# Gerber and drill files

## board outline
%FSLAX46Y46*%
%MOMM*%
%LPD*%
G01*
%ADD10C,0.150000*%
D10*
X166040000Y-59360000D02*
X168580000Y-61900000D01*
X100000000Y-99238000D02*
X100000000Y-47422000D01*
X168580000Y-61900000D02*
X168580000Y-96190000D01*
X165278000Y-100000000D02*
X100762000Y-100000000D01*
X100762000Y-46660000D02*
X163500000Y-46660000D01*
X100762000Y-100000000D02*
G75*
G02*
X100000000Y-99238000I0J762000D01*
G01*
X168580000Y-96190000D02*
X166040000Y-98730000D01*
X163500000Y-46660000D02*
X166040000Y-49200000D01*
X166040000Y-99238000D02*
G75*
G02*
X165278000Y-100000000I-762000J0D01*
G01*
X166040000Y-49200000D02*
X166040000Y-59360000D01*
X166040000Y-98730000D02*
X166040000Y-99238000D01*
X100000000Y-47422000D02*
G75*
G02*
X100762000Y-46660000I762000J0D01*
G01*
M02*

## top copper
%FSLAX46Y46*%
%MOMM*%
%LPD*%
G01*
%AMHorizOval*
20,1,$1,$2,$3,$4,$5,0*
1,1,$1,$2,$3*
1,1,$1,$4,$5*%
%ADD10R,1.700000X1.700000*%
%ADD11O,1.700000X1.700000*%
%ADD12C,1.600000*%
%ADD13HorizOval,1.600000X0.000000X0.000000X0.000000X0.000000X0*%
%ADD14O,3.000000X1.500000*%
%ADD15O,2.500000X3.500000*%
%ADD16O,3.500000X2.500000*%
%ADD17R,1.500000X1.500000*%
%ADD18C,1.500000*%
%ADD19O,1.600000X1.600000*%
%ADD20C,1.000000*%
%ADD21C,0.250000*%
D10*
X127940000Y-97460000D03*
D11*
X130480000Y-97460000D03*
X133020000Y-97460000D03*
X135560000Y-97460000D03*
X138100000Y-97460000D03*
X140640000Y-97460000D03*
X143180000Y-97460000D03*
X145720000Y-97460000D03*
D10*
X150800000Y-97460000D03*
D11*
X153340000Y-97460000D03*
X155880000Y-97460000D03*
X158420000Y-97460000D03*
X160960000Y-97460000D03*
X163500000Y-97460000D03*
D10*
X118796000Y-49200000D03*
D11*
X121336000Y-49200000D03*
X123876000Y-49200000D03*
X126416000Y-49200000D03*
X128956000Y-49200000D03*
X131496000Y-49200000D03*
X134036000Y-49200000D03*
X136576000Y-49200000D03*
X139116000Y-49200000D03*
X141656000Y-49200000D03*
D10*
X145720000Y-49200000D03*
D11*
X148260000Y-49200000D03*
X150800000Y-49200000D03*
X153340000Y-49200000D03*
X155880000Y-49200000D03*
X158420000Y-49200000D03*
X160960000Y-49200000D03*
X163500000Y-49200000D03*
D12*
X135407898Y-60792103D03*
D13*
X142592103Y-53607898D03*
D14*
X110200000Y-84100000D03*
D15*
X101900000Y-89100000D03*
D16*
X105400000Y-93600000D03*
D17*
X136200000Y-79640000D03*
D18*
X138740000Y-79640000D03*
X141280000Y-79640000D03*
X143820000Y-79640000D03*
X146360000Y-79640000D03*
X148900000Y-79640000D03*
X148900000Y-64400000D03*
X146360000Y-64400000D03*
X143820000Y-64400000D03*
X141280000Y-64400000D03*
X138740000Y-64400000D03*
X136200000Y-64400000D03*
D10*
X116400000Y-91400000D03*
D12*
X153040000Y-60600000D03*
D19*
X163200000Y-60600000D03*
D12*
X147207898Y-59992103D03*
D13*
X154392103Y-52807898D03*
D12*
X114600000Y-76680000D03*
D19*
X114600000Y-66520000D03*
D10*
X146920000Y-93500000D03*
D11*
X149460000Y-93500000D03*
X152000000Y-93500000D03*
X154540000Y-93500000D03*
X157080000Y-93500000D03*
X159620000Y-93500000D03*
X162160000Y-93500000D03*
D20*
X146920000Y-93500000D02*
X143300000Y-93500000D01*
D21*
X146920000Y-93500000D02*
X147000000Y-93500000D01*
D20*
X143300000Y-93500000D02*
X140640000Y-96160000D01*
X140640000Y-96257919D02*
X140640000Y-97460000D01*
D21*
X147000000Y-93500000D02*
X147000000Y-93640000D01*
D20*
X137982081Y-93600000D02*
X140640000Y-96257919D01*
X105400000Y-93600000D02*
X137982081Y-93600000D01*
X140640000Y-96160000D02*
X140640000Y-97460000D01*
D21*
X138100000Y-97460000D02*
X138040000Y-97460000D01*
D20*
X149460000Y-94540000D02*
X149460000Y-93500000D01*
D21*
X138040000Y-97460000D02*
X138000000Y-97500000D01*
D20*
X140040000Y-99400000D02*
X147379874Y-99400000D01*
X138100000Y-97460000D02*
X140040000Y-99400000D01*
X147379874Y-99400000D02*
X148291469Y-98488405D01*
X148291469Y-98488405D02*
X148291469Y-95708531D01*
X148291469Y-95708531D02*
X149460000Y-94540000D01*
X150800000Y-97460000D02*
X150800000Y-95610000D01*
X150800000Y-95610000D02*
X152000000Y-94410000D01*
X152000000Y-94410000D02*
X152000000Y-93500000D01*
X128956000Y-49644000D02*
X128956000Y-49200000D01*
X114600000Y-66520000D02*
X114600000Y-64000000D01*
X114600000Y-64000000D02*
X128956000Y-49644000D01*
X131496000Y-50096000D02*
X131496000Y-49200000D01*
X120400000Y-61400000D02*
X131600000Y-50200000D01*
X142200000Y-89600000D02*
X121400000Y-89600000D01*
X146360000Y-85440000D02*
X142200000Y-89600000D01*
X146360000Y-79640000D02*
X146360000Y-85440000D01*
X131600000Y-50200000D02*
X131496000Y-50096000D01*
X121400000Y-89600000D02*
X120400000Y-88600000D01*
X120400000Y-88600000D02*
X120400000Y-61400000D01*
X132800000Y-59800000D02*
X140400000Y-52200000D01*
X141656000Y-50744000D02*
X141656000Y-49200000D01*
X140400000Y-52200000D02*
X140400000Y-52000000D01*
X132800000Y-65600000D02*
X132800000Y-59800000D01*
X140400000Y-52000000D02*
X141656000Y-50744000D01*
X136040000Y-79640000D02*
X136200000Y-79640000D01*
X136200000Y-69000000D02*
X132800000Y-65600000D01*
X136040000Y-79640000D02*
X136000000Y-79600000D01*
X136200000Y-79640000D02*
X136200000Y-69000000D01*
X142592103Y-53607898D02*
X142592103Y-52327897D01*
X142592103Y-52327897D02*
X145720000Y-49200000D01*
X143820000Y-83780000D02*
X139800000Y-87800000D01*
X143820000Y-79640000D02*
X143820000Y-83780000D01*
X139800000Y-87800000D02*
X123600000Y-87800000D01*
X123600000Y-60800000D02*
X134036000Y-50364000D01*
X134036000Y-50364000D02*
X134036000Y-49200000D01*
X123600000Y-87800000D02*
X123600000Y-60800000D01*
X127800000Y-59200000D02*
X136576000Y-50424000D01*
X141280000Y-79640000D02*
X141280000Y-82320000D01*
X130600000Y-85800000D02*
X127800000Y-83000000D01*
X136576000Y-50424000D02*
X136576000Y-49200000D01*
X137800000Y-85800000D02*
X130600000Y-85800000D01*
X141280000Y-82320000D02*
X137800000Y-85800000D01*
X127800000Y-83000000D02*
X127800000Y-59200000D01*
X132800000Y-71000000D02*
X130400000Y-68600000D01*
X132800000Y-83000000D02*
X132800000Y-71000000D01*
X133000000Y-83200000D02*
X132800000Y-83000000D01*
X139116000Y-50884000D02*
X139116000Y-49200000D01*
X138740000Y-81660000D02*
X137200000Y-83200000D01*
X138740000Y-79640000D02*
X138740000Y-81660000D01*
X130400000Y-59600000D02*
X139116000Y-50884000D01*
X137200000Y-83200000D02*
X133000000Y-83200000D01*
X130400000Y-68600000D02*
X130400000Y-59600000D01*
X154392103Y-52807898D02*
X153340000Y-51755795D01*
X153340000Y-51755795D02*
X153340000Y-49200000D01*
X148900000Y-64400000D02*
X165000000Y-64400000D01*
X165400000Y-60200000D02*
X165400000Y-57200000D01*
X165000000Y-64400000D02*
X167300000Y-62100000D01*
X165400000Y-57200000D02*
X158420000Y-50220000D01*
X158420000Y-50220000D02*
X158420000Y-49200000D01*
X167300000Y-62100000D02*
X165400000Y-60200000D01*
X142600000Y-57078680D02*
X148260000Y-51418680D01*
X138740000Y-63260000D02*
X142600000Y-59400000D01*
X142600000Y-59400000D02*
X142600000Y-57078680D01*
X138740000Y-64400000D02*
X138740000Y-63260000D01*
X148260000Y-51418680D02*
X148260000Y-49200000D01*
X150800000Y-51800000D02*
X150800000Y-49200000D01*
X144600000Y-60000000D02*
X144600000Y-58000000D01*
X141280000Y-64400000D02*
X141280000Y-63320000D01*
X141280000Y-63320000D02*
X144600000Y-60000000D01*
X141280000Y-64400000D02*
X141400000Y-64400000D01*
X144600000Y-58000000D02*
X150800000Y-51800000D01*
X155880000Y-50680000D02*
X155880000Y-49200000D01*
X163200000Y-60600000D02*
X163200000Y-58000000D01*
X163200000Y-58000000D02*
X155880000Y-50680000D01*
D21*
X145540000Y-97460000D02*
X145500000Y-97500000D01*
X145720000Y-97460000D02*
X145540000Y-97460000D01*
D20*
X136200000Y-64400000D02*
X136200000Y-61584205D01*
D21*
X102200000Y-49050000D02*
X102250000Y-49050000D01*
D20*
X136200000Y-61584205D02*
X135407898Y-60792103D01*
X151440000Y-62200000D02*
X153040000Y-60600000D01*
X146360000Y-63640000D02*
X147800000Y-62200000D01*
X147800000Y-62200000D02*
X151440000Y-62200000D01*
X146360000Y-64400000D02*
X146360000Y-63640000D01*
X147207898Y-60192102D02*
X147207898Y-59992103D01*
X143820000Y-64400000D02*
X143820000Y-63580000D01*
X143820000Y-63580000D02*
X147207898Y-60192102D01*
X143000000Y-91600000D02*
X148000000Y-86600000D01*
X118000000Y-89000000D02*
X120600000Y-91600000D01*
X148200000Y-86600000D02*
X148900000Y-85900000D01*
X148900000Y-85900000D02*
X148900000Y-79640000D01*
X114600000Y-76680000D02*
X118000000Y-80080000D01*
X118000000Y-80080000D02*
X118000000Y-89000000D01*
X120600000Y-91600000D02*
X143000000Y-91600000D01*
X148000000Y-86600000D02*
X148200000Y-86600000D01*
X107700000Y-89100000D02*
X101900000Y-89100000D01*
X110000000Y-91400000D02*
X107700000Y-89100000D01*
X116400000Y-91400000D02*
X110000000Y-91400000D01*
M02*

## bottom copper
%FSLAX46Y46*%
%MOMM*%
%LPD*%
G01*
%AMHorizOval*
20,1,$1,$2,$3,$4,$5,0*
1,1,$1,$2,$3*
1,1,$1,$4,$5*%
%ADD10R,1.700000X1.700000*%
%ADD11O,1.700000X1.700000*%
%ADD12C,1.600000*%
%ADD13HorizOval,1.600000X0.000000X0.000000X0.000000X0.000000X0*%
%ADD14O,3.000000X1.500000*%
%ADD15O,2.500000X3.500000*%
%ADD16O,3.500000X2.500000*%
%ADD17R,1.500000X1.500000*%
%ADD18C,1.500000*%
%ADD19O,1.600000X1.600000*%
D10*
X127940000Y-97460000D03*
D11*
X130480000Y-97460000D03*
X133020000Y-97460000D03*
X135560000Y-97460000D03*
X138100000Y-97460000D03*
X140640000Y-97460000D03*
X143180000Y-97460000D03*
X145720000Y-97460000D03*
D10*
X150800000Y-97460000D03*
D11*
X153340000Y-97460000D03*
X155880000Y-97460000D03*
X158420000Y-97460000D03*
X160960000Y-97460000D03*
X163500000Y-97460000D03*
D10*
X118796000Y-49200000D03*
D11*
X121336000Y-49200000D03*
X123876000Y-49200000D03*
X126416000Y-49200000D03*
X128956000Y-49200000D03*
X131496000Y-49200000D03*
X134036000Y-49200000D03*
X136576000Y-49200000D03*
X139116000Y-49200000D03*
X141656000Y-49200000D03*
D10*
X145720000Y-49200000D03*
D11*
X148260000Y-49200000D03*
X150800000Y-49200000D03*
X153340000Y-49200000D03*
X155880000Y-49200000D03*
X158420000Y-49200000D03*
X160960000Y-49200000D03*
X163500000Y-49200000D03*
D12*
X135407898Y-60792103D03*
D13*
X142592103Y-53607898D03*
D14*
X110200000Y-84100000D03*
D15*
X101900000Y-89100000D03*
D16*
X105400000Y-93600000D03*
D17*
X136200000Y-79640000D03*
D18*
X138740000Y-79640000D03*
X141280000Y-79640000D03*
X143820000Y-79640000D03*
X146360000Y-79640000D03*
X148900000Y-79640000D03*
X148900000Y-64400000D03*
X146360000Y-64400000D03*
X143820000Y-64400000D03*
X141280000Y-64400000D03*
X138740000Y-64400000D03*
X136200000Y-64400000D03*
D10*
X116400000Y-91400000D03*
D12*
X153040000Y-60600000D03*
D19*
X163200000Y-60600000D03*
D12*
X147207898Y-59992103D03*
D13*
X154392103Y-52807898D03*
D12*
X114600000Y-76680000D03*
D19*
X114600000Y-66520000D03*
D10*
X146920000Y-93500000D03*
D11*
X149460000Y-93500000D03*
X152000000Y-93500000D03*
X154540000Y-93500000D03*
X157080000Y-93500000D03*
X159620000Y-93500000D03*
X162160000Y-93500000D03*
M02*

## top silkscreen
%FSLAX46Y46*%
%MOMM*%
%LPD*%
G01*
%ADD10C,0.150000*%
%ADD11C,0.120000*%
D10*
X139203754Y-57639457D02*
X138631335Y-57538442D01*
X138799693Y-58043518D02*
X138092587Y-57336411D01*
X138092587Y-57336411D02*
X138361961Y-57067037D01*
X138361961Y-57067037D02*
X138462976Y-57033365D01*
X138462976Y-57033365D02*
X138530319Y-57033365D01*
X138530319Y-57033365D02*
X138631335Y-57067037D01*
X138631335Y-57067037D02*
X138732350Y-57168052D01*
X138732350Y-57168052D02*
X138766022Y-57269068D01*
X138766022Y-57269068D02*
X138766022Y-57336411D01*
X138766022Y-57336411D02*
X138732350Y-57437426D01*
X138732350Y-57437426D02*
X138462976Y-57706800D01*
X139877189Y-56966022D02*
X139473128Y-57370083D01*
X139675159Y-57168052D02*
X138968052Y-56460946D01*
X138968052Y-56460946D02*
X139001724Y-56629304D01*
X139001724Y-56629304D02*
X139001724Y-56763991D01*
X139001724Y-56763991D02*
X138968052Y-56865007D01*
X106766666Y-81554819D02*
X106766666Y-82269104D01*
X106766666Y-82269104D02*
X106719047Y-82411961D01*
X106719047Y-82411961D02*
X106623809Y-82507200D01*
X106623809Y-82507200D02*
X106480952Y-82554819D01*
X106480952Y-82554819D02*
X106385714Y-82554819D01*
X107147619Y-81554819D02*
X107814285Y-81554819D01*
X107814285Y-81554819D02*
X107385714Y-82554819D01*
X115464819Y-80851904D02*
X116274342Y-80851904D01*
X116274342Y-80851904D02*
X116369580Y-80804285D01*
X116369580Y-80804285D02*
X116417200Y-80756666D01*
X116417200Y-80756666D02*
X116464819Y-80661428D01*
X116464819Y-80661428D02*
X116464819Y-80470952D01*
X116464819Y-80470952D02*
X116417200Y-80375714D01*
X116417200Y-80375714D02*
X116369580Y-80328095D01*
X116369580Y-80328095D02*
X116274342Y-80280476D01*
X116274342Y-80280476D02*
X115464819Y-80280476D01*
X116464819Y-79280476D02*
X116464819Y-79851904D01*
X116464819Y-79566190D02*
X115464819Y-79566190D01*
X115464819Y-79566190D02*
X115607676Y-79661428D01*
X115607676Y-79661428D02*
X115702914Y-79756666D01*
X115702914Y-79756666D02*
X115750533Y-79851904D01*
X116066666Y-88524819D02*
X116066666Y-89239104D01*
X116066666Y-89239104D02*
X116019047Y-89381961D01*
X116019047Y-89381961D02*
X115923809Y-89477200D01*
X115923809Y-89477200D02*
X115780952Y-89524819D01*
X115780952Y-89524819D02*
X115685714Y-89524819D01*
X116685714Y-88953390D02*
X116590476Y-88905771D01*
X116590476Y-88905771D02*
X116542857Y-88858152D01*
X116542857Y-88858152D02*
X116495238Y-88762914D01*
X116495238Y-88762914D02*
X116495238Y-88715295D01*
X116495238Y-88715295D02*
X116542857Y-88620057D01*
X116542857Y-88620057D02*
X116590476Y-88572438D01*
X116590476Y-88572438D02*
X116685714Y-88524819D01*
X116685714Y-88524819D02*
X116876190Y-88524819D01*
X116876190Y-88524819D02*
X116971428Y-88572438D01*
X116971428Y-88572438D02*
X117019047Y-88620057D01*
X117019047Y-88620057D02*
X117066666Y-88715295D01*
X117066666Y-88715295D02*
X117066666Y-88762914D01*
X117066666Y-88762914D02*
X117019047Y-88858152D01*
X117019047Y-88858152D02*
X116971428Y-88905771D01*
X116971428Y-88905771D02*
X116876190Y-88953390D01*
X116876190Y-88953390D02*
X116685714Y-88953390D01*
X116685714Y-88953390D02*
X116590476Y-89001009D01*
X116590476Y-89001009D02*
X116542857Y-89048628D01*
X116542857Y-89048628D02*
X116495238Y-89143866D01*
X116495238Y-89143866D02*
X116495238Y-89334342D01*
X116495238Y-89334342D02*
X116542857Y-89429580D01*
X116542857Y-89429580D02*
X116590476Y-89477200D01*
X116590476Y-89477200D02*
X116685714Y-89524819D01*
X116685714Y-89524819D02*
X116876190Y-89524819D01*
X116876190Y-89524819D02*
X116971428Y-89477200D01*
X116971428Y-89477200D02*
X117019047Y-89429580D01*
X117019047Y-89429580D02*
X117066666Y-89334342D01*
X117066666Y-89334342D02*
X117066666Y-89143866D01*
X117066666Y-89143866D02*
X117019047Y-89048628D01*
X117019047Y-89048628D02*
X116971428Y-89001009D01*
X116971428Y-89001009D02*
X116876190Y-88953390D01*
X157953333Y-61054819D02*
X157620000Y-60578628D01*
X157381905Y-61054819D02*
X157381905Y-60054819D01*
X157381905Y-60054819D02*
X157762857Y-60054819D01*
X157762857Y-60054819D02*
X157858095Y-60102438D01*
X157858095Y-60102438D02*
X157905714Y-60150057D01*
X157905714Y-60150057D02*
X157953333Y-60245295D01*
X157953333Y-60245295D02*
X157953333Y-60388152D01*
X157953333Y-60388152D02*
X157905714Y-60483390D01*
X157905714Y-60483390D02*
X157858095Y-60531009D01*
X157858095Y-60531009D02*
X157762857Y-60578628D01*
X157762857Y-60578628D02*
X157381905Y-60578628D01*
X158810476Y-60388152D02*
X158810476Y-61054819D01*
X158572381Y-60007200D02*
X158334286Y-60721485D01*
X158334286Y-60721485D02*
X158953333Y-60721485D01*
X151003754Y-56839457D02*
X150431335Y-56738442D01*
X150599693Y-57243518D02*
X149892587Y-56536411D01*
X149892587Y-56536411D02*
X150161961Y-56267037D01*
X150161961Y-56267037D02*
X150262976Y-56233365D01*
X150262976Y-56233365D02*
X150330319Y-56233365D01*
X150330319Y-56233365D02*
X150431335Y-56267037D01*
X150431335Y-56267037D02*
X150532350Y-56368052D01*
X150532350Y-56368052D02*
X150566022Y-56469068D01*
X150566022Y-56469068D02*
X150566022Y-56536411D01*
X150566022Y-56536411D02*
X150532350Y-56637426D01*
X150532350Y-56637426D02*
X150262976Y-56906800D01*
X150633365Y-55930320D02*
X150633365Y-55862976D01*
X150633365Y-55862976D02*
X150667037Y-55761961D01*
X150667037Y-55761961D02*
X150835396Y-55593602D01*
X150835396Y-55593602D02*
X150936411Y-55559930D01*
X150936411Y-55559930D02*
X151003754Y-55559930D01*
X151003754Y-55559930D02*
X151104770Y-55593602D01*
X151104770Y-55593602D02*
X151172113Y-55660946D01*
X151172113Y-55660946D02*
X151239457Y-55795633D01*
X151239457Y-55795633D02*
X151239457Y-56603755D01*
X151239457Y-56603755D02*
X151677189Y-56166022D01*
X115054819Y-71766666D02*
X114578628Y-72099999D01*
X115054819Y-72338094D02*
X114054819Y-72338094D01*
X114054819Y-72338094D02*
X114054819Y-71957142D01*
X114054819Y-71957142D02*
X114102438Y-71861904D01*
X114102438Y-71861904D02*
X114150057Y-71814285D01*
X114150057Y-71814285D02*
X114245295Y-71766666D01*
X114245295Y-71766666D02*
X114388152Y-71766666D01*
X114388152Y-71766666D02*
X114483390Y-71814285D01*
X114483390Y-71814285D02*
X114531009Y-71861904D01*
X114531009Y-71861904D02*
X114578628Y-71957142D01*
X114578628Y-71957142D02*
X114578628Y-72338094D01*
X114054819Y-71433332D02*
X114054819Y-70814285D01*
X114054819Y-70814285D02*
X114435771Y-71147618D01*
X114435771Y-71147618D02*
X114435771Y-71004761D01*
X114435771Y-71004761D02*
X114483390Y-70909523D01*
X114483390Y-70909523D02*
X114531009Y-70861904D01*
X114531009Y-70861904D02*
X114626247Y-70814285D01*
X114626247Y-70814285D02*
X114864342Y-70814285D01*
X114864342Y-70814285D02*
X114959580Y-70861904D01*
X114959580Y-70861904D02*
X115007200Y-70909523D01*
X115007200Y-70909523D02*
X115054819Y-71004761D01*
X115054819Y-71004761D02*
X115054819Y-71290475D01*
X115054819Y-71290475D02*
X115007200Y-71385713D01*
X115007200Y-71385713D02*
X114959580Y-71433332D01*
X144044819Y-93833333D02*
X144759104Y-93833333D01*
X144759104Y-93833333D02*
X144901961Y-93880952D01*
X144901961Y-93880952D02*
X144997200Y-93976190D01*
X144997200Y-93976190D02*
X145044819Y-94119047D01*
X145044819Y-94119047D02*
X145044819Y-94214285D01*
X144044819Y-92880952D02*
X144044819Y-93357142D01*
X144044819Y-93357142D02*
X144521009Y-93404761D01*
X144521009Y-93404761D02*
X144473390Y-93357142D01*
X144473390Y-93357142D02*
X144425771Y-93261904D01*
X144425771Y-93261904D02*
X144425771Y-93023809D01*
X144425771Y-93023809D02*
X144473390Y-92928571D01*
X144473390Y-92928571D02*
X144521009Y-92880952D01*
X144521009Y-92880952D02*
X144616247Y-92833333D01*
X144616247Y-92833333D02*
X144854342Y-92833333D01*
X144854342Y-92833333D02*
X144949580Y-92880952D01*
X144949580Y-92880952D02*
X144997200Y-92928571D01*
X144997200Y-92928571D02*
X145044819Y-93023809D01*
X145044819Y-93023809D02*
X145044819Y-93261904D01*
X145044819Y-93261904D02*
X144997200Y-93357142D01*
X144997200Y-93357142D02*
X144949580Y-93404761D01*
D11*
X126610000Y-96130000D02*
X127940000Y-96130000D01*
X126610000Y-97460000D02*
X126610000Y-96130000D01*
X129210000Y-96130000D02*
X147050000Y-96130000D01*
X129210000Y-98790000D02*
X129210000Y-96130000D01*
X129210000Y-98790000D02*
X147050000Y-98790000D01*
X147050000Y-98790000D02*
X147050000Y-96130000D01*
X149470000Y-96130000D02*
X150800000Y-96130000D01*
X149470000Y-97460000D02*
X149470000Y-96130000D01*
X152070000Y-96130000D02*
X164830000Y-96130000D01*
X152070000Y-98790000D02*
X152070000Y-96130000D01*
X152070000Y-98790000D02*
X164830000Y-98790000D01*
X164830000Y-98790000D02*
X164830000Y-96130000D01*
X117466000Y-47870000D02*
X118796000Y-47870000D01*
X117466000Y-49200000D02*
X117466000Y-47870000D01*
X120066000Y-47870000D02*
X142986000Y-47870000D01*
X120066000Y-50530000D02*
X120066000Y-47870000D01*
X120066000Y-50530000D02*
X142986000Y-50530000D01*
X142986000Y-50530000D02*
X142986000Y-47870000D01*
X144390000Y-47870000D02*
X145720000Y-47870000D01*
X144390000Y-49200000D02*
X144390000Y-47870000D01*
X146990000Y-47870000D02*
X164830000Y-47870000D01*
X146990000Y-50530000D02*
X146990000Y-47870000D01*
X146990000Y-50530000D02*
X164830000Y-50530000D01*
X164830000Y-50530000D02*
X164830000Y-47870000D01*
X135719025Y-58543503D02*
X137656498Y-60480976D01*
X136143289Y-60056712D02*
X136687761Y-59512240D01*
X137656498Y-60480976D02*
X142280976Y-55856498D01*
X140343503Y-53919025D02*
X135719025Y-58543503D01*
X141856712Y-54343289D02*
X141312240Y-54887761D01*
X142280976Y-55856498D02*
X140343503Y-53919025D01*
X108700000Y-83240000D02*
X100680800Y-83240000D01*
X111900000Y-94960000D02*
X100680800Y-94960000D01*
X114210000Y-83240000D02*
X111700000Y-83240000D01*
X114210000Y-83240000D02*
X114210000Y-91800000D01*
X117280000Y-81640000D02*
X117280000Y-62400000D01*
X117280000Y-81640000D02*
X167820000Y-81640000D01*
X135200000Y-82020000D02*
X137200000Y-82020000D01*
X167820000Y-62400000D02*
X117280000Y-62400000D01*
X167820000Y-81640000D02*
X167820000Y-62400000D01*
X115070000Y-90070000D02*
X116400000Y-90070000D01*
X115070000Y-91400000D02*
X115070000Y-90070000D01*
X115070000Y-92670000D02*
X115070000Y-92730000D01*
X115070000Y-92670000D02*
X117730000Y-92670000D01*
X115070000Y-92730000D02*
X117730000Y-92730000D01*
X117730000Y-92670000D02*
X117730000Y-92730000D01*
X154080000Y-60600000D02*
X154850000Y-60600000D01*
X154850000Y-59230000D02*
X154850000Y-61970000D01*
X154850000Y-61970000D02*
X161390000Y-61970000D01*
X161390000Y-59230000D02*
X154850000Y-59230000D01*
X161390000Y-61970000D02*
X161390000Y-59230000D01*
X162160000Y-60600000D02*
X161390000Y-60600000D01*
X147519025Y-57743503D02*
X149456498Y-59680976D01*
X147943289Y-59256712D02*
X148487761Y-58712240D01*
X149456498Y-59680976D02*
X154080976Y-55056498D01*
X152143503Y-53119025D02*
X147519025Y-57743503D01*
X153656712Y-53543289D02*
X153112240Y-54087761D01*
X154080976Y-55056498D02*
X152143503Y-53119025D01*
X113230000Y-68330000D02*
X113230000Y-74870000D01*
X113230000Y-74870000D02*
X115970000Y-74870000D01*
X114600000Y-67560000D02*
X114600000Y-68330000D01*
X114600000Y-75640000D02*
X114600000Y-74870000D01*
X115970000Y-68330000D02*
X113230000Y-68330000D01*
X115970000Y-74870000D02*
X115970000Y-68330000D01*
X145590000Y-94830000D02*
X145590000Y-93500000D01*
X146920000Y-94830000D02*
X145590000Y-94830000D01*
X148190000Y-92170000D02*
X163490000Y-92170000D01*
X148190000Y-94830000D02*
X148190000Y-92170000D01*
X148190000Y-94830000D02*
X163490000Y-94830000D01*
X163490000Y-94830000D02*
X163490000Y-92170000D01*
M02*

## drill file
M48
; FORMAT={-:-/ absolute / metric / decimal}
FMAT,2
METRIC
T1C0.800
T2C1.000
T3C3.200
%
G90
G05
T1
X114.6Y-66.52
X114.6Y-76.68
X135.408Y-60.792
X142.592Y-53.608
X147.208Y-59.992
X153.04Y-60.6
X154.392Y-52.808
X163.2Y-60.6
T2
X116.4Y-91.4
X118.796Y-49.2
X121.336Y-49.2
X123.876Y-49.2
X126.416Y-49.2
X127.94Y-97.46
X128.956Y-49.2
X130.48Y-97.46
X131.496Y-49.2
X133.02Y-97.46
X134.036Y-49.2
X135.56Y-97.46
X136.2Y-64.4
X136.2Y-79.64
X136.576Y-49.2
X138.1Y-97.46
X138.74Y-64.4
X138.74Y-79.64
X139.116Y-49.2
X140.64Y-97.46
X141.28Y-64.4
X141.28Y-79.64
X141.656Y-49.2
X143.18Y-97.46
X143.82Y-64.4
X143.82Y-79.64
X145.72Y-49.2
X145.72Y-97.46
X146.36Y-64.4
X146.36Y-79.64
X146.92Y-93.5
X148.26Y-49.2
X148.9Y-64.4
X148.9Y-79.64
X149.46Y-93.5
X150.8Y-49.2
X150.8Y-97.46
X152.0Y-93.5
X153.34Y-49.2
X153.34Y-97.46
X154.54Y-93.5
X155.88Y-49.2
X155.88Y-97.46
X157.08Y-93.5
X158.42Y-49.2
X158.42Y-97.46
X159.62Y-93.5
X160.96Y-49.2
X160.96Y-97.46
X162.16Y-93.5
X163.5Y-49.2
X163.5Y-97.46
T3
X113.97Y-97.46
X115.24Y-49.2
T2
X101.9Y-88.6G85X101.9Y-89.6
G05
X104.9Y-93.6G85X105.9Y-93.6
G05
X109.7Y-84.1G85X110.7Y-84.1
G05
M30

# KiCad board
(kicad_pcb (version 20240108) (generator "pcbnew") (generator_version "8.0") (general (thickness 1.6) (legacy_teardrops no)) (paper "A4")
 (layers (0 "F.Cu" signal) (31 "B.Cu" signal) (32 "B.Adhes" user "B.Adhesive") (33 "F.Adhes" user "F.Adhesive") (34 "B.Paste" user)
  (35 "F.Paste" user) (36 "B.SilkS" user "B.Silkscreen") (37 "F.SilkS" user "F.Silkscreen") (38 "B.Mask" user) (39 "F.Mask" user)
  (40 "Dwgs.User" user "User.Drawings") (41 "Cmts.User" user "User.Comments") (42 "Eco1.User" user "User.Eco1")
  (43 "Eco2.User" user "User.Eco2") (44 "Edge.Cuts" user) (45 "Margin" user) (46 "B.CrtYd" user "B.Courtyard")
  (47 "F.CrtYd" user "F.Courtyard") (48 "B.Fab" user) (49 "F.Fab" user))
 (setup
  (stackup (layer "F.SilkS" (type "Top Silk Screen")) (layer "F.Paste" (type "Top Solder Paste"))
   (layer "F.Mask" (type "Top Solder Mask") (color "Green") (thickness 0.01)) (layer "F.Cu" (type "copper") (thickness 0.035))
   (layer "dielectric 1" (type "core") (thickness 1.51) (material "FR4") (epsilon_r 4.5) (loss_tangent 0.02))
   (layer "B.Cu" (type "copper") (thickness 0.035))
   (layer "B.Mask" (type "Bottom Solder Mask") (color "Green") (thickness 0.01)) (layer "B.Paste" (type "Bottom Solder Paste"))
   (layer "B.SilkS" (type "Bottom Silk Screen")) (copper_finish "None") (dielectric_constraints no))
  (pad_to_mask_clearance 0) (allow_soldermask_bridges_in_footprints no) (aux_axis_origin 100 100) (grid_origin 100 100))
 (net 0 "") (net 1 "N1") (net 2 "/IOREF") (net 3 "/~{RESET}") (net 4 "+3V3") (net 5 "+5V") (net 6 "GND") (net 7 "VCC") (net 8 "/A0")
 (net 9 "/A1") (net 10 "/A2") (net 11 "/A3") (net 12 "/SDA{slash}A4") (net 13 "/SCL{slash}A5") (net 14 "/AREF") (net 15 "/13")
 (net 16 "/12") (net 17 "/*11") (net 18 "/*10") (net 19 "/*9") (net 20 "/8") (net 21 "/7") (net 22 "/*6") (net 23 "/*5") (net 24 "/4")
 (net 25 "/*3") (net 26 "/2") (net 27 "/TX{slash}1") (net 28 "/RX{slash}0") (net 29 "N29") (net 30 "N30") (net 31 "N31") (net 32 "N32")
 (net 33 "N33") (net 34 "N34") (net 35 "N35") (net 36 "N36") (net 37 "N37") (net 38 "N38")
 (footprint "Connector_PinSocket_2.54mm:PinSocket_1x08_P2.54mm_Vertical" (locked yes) (layer "F.Cu") (at 127.94 97.46 90)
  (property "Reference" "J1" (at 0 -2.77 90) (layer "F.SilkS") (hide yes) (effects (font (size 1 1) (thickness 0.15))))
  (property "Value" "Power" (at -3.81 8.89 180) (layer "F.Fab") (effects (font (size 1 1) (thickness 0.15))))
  (fp_line (start 1.33 -1.33) (end 1.33 0) (stroke (width 0.12) (type solid)) (layer "F.SilkS"))
  (fp_line (start 0 -1.33) (end 1.33 -1.33) (stroke (width 0.12) (type solid)) (layer "F.SilkS"))
  (fp_line (start 1.33 1.27) (end 1.33 19.11) (stroke (width 0.12) (type solid)) (layer "F.SilkS"))
  (fp_line (start -1.33 1.27) (end 1.33 1.27) (stroke (width 0.12) (type solid)) (layer "F.SilkS"))
  (fp_line (start -1.33 1.27) (end -1.33 19.11) (stroke (width 0.12) (type solid)) (layer "F.SilkS"))
  (fp_line (start -1.33 19.11) (end 1.33 19.11) (stroke (width 0.12) (type solid)) (layer "F.SilkS"))
  (pad "1" thru_hole rect (at 0 0 90) (size 1.7 1.7) (drill 1) (layers "*.Cu" "*.Mask") (remove_unused_layers no) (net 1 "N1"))
  (pad "2" thru_hole oval (at 0 2.54 90) (size 1.7 1.7) (drill 1) (layers "*.Cu" "*.Mask") (remove_unused_layers no) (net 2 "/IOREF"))
  (pad "3" thru_hole oval (at 0 5.08 90) (size 1.7 1.7) (drill 1) (layers "*.Cu" "*.Mask") (remove_unused_layers no) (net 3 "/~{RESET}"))
  (pad "4" thru_hole oval (at 0 7.62 90) (size 1.7 1.7) (drill 1) (layers "*.Cu" "*.Mask") (remove_unused_layers no) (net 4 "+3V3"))
  (pad "5" thru_hole oval (at 0 10.16 90) (size 1.7 1.7) (drill 1) (layers "*.Cu" "*.Mask") (remove_unused_layers no) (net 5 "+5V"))
  (pad "6" thru_hole oval (at 0 12.7 90) (size 1.7 1.7) (drill 1) (layers "*.Cu" "*.Mask") (remove_unused_layers no) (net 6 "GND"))
  (pad "7" thru_hole oval (at 0 15.24 90) (size 1.7 1.7) (drill 1) (layers "*.Cu" "*.Mask") (remove_unused_layers no) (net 6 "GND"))
  (pad "8" thru_hole oval (at 0 17.78 90) (size 1.7 1.7) (drill 1) (layers "*.Cu" "*.Mask") (remove_unused_layers no) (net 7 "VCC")))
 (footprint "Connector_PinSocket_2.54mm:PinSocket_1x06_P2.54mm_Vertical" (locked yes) (layer "F.Cu") (at 150.8 97.46 90)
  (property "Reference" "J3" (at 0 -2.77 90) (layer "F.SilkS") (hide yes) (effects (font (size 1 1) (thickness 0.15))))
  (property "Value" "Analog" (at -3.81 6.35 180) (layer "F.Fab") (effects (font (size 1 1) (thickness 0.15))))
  (fp_line (start 1.33 -1.33) (end 1.33 0) (stroke (width 0.12) (type solid)) (layer "F.SilkS"))
  (fp_line (start 0 -1.33) (end 1.33 -1.33) (stroke (width 0.12) (type solid)) (layer "F.SilkS"))
  (fp_line (start 1.33 1.27) (end 1.33 14.03) (stroke (width 0.12) (type solid)) (layer "F.SilkS"))
  (fp_line (start -1.33 1.27) (end 1.33 1.27) (stroke (width 0.12) (type solid)) (layer "F.SilkS"))
  (fp_line (start -1.33 1.27) (end -1.33 14.03) (stroke (width 0.12) (type solid)) (layer "F.SilkS"))
  (fp_line (start -1.33 14.03) (end 1.33 14.03) (stroke (width 0.12) (type solid)) (layer "F.SilkS"))
  (pad "1" thru_hole rect (at 0 0 90) (size 1.7 1.7) (drill 1) (layers "*.Cu" "*.Mask") (remove_unused_layers no) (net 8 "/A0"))
  (pad "2" thru_hole oval (at 0 2.54 90) (size 1.7 1.7) (drill 1) (layers "*.Cu" "*.Mask") (remove_unused_layers no) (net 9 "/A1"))
  (pad "3" thru_hole oval (at 0 5.08 90) (size 1.7 1.7) (drill 1) (layers "*.Cu" "*.Mask") (remove_unused_layers no) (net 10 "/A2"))
  (pad "4" thru_hole oval (at 0 7.62 90) (size 1.7 1.7) (drill 1) (layers "*.Cu" "*.Mask") (remove_unused_layers no) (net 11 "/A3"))
  (pad "5" thru_hole oval (at 0 10.16 90) (size 1.7 1.7) (drill 1) (layers "*.Cu" "*.Mask") (remove_unused_layers no)
   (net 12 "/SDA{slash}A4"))
  (pad "6" thru_hole oval (at 0 12.7 90) (size 1.7 1.7) (drill 1) (layers "*.Cu" "*.Mask") (remove_unused_layers no)
   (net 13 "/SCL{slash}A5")))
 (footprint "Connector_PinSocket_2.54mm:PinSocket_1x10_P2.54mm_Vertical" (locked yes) (layer "F.Cu") (at 118.796 49.2 90)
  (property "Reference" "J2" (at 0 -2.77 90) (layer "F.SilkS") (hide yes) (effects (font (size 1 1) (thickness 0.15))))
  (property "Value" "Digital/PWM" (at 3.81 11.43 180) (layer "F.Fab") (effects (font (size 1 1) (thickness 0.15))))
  (fp_line (start 1.33 -1.33) (end 1.33 0) (stroke (width 0.12) (type solid)) (layer "F.SilkS"))
  (fp_line (start 0 -1.33) (end 1.33 -1.33) (stroke (width 0.12) (type solid)) (layer "F.SilkS"))
  (fp_line (start 1.33 1.27) (end 1.33 24.19) (stroke (width 0.12) (type solid)) (layer "F.SilkS"))
  (fp_line (start -1.33 1.27) (end 1.33 1.27) (stroke (width 0.12) (type solid)) (layer "F.SilkS"))
  (fp_line (start -1.33 1.27) (end -1.33 24.19) (stroke (width 0.12) (type solid)) (layer "F.SilkS"))
  (fp_line (start -1.33 24.19) (end 1.33 24.19) (stroke (width 0.12) (type solid)) (layer "F.SilkS"))
  (pad "1" thru_hole rect (at 0 0 90) (size 1.7 1.7) (drill 1) (layers "*.Cu" "*.Mask") (remove_unused_layers no) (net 13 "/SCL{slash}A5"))
  (pad "2" thru_hole oval (at 0 2.54 90) (size 1.7 1.7) (drill 1) (layers "*.Cu" "*.Mask") (remove_unused_layers no)
   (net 12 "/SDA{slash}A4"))
  (pad "3" thru_hole oval (at 0 5.08 90) (size 1.7 1.7) (drill 1) (layers "*.Cu" "*.Mask") (remove_unused_layers no) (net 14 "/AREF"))
  (pad "4" thru_hole oval (at 0 7.62 90) (size 1.7 1.7) (drill 1) (layers "*.Cu" "*.Mask") (remove_unused_layers no) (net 6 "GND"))
  (pad "5" thru_hole oval (at 0 10.16 90) (size 1.7 1.7) (drill 1) (layers "*.Cu" "*.Mask") (remove_unused_layers no) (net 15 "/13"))
  (pad "6" thru_hole oval (at 0 12.7 90) (size 1.7 1.7) (drill 1) (layers "*.Cu" "*.Mask") (remove_unused_layers no) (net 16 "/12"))
  (pad "7" thru_hole oval (at 0 15.24 90) (size 1.7 1.7) (drill 1) (layers "*.Cu" "*.Mask") (remove_unused_layers no) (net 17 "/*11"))
  (pad "8" thru_hole oval (at 0 17.78 90) (size 1.7 1.7) (drill 1) (layers "*.Cu" "*.Mask") (remove_unused_layers no) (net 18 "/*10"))
  (pad "9" thru_hole oval (at 0 20.32 90) (size 1.7 1.7) (drill 1) (layers "*.Cu" "*.Mask") (remove_unused_layers no) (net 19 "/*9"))
  (pad "10" thru_hole oval (at 0 22.86 90) (size 1.7 1.7) (drill 1) (layers "*.Cu" "*.Mask") (remove_unused_layers no) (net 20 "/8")))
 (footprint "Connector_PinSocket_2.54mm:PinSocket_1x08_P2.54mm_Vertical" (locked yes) (layer "F.Cu") (at 145.72 49.2 90)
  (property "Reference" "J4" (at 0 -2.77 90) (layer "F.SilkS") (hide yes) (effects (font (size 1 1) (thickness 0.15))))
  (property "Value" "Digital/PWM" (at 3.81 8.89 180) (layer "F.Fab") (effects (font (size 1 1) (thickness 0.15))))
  (fp_line (start 1.33 -1.33) (end 1.33 0) (stroke (width 0.12) (type solid)) (layer "F.SilkS"))
  (fp_line (start 0 -1.33) (end 1.33 -1.33) (stroke (width 0.12) (type solid)) (layer "F.SilkS"))
  (fp_line (start 1.33 1.27) (end 1.33 19.11) (stroke (width 0.12) (type solid)) (layer "F.SilkS"))
  (fp_line (start -1.33 1.27) (end 1.33 1.27) (stroke (width 0.12) (type solid)) (layer "F.SilkS"))
  (fp_line (start -1.33 1.27) (end -1.33 19.11) (stroke (width 0.12) (type solid)) (layer "F.SilkS"))
  (fp_line (start -1.33 19.11) (end 1.33 19.11) (stroke (width 0.12) (type solid)) (layer "F.SilkS"))
  (pad "1" thru_hole rect (at 0 0 90) (size 1.7 1.7) (drill 1) (layers "*.Cu" "*.Mask") (remove_unused_layers no) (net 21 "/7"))
  (pad "2" thru_hole oval (at 0 2.54 90) (size 1.7 1.7) (drill 1) (layers "*.Cu" "*.Mask") (remove_unused_layers no) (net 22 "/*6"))
  (pad "3" thru_hole oval (at 0 5.08 90) (size 1.7 1.7) (drill 1) (layers "*.Cu" "*.Mask") (remove_unused_layers no) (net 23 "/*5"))
  (pad "4" thru_hole oval (at 0 7.62 90) (size 1.7 1.7) (drill 1) (layers "*.Cu" "*.Mask") (remove_unused_layers no) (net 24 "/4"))
  (pad "5" thru_hole oval (at 0 10.16 90) (size 1.7 1.7) (drill 1) (layers "*.Cu" "*.Mask") (remove_unused_layers no) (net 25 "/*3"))
  (pad "6" thru_hole oval (at 0 12.7 90) (size 1.7 1.7) (drill 1) (layers "*.Cu" "*.Mask") (remove_unused_layers no) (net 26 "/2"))
  (pad "7" thru_hole oval (at 0 15.24 90) (size 1.7 1.7) (drill 1) (layers "*.Cu" "*.Mask") (remove_unused_layers no) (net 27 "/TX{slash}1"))
  (pad "8" thru_hole oval (at 0 17.78 90) (size 1.7 1.7) (drill 1) (layers "*.Cu" "*.Mask") (remove_unused_layers no) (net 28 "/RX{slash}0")))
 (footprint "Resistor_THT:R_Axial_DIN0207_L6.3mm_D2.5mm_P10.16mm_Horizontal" (layer "F.Cu") (at 135.407898 60.792103 45)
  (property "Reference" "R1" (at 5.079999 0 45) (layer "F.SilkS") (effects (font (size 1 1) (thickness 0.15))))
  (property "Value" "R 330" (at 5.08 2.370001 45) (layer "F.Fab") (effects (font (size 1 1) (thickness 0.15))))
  (fp_line (start 1.81 -1.37) (end 1.81 1.37) (stroke (width 0.12) (type solid)) (layer "F.SilkS"))
  (fp_line (start 1.04 0) (end 1.81 0) (stroke (width 0.12) (type solid)) (layer "F.SilkS"))
  (fp_line (start 1.81 1.37) (end 8.35 1.37) (stroke (width 0.12) (type solid)) (layer "F.SilkS"))
  (fp_line (start 8.35 -1.37) (end 1.81 -1.37) (stroke (width 0.12) (type solid)) (layer "F.SilkS"))
  (fp_line (start 9.12 0) (end 8.350001 0) (stroke (width 0.12) (type solid)) (layer "F.SilkS"))
  (fp_line (start 8.35 1.37) (end 8.35 -1.37) (stroke (width 0.12) (type solid)) (layer "F.SilkS"))
  (pad "1" thru_hole circle (at 0 0 45) (size 1.6 1.6) (drill 0.8) (layers "*.Cu" "*.Mask") (remove_unused_layers no) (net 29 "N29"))
  (pad "2" thru_hole oval (at 10.16 0 45) (size 1.6 1.6) (drill 0.8) (layers "*.Cu" "*.Mask") (remove_unused_layers no) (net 21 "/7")))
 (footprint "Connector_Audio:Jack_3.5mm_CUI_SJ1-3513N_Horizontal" (layer "F.Cu") (at 101.9 89.1)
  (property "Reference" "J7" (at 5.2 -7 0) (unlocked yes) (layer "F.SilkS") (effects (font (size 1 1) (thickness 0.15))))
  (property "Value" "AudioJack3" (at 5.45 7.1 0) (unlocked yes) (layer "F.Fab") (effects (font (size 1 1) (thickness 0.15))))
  (fp_line (start 6.8 -5.86) (end -1.2192 -5.86) (stroke (width 0.12) (type solid)) (layer "F.SilkS"))
  (fp_line (start 10 5.86) (end -1.2192 5.86) (stroke (width 0.12) (type solid)) (layer "F.SilkS"))
  (fp_line (start 12.31 -5.86) (end 9.8 -5.86) (stroke (width 0.12) (type solid)) (layer "F.SilkS"))
  (fp_line (start 12.31 -5.86) (end 12.31 2.7) (stroke (width 0.12) (type solid)) (layer "F.SilkS"))
  (pad "R" thru_hole oval (at 8.3 -5) (size 3 1.5) (drill oval 2 1) (layers "*.Cu" "*.Mask") (remove_unused_layers no) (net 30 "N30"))
  (pad "S" thru_hole oval (at 0 0 270) (size 3.5 2.5) (drill oval 2 1) (layers "*.Cu" "*.Mask") (remove_unused_layers no) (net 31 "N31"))
  (pad "T" thru_hole oval (at 3.5 4.5) (size 3.5 2.5) (drill oval 2 1) (layers "*.Cu" "*.Mask") (remove_unused_layers no) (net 6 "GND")))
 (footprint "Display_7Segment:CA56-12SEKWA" (layer "F.Cu") (at 136.2 79.64 90)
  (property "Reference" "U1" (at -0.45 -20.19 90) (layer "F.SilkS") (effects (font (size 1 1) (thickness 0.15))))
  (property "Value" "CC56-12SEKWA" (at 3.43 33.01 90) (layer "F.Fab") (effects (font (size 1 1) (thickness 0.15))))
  (fp_line (start -2 -18.92) (end 17.24 -18.92) (stroke (width 0.12) (type solid)) (layer "F.SilkS"))
  (fp_line (start -2 -18.92) (end -2 31.62) (stroke (width 0.12) (type solid)) (layer "F.SilkS"))
  (fp_line (start -2.38 -1) (end -2.38 1) (stroke (width 0.12) (type solid)) (layer "F.SilkS"))
  (fp_line (start 17.24 31.62) (end 17.24 -18.92) (stroke (width 0.12) (type solid)) (layer "F.SilkS"))
  (fp_line (start -2 31.62) (end 17.24 31.62) (stroke (width 0.12) (type solid)) (layer "F.SilkS"))
  (pad "1" thru_hole rect (at 0 0 90) (size 1.5 1.5) (drill 1) (layers "*.Cu" "*.Mask") (remove_unused_layers no) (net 20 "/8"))
  (pad "2" thru_hole circle (at 0 2.54 90) (size 1.5 1.5) (drill 1) (layers "*.Cu" "*.Mask") (remove_unused_layers no) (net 19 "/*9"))
  (pad "3" thru_hole circle (at 0 5.08 90) (size 1.5 1.5) (drill 1) (layers "*.Cu" "*.Mask") (remove_unused_layers no) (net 18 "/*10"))
  (pad "4" thru_hole circle (at 0 7.62 90) (size 1.5 1.5) (drill 1) (layers "*.Cu" "*.Mask") (remove_unused_layers no) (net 17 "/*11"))
  (pad "5" thru_hole circle (at 0 10.16 90) (size 1.5 1.5) (drill 1) (layers "*.Cu" "*.Mask") (remove_unused_layers no) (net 16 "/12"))
  (pad "6" thru_hole circle (at 0 12.7 90) (size 1.5 1.5) (drill 1) (layers "*.Cu" "*.Mask") (remove_unused_layers no) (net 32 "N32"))
  (pad "7" thru_hole circle (at 15.24 12.7 90) (size 1.5 1.5) (drill 1) (layers "*.Cu" "*.Mask") (remove_unused_layers no) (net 26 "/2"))
  (pad "8" thru_hole circle (at 15.24 10.16 90) (size 1.5 1.5) (drill 1) (layers "*.Cu" "*.Mask") (remove_unused_layers no) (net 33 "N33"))
  (pad "9" thru_hole circle (at 15.24 7.62 90) (size 1.5 1.5) (drill 1) (layers "*.Cu" "*.Mask") (remove_unused_layers no) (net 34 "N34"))
  (pad "10" thru_hole circle (at 15.24 5.08 90) (size 1.5 1.5) (drill 1) (layers "*.Cu" "*.Mask") (remove_unused_layers no) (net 23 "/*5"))
  (pad "11" thru_hole circle (at 15.24 2.54 90) (size 1.5 1.5) (drill 1) (layers "*.Cu" "*.Mask") (remove_unused_layers no) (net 22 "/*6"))
  (pad "12" thru_hole circle (at 15.24 0 90) (size 1.5 1.5) (drill 1) (layers "*.Cu" "*.Mask") (remove_unused_layers no) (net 29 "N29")))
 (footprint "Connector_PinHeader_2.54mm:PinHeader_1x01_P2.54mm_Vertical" (layer "F.Cu") (at 116.4 91.4)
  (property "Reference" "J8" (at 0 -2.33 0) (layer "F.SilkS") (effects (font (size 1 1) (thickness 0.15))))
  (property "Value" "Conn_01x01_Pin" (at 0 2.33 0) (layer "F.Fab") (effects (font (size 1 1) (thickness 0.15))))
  (fp_line (start -1.33 -1.33) (end 0 -1.33) (stroke (width 0.12) (type solid)) (layer "F.SilkS"))
  (fp_line (start -1.33 0) (end -1.33 -1.33) (stroke (width 0.12) (type solid)) (layer "F.SilkS"))
  (fp_line (start -1.33 1.27) (end -1.33 1.33) (stroke (width 0.12) (type solid)) (layer "F.SilkS"))
  (fp_line (start -1.33 1.27) (end 1.33 1.27) (stroke (width 0.12) (type solid)) (layer "F.SilkS"))
  (fp_line (start -1.33 1.33) (end 1.33 1.33) (stroke (width 0.12) (type solid)) (layer "F.SilkS"))
  (fp_line (start 1.33 1.27) (end 1.33 1.33) (stroke (width 0.12) (type solid)) (layer "F.SilkS"))
  (pad "1" thru_hole rect (at 0 0) (size 1.7 1.7) (drill 1) (layers "*.Cu" "*.Mask") (remove_unused_layers no) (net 31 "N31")))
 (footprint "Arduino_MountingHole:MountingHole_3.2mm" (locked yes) (layer "F.Cu") (at 115.24 49.2)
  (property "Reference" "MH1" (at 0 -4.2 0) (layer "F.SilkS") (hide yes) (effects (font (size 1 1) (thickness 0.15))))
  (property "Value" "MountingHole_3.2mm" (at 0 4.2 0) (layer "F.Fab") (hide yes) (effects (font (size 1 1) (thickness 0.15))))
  (pad "" np_thru_hole circle (at 0 0) (size 3.2 3.2) (drill 3.2) (layers "*.Cu" "*.Mask")))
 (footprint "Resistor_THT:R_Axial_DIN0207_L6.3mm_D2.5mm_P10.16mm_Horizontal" (layer "F.Cu") (at 153.04 60.6)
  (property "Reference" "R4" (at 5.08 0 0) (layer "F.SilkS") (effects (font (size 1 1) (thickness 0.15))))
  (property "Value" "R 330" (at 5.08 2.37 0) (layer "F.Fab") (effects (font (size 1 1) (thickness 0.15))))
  (fp_line (start 1.04 0) (end 1.81 0) (stroke (width 0.12) (type solid)) (layer "F.SilkS"))
  (fp_line (start 1.81 -1.37) (end 1.81 1.37) (stroke (width 0.12) (type solid)) (layer "F.SilkS"))
  (fp_line (start 1.81 1.37) (end 8.35 1.37) (stroke (width 0.12) (type solid)) (layer "F.SilkS"))
  (fp_line (start 8.35 -1.37) (end 1.81 -1.37) (stroke (width 0.12) (type solid)) (layer "F.SilkS"))
  (fp_line (start 8.35 1.37) (end 8.35 -1.37) (stroke (width 0.12) (type solid)) (layer "F.SilkS"))
  (fp_line (start 9.12 0) (end 8.35 0) (stroke (width 0.12) (type solid)) (layer "F.SilkS"))
  (pad "1" thru_hole circle (at 0 0) (size 1.6 1.6) (drill 0.8) (layers "*.Cu" "*.Mask") (remove_unused_layers no) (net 33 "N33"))
  (pad "2" thru_hole oval (at 10.16 0) (size 1.6 1.6) (drill 0.8) (layers "*.Cu" "*.Mask") (remove_unused_layers no) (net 25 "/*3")))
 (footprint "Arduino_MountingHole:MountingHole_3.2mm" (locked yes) (layer "F.Cu") (at 113.97 97.46)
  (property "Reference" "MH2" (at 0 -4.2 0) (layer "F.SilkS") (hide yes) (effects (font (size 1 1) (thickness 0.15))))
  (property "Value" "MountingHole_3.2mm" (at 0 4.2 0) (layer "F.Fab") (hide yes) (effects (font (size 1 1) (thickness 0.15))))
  (pad "" np_thru_hole circle (at 0 0) (size 3.2 3.2) (drill 3.2) (layers "*.Cu" "*.Mask")))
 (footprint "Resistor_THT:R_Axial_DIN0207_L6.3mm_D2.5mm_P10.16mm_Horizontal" (layer "F.Cu") (at 147.207898 59.992103 45)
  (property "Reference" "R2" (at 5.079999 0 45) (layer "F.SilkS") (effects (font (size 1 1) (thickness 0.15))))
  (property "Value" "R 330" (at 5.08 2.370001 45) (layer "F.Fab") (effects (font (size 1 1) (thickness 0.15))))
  (fp_line (start 1.81 -1.37) (end 1.81 1.37) (stroke (width 0.12) (type solid)) (layer "F.SilkS"))
  (fp_line (start 1.04 0) (end 1.81 0) (stroke (width 0.12) (type solid)) (layer "F.SilkS"))
  (fp_line (start 1.81 1.37) (end 8.35 1.37) (stroke (width 0.12) (type solid)) (layer "F.SilkS"))
  (fp_line (start 8.35 -1.37) (end 1.81 -1.37) (stroke (width 0.12) (type solid)) (layer "F.SilkS"))
  (fp_line (start 9.12 0) (end 8.350001 0) (stroke (width 0.12) (type solid)) (layer "F.SilkS"))
  (fp_line (start 8.35 1.37) (end 8.35 -1.37) (stroke (width 0.12) (type solid)) (layer "F.SilkS"))
  (pad "1" thru_hole circle (at 0 0 45) (size 1.6 1.6) (drill 0.8) (layers "*.Cu" "*.Mask") (remove_unused_layers no) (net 34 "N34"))
  (pad "2" thru_hole oval (at 10.16 0 45) (size 1.6 1.6) (drill 0.8) (layers "*.Cu" "*.Mask") (remove_unused_layers no) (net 24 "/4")))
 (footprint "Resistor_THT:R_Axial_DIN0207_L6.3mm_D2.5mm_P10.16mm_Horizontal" (layer "F.Cu") (at 114.6 76.68 90)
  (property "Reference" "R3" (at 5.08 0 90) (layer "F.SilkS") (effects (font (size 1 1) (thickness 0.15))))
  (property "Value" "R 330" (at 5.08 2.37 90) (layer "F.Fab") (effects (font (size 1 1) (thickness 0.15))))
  (fp_line (start 8.35 -1.37) (end 1.81 -1.37) (stroke (width 0.12) (type solid)) (layer "F.SilkS"))
  (fp_line (start 1.81 -1.37) (end 1.81 1.37) (stroke (width 0.12) (type solid)) (layer "F.SilkS"))
  (fp_line (start 9.12 0) (end 8.35 0) (stroke (width 0.12) (type solid)) (layer "F.SilkS"))
  (fp_line (start 1.04 0) (end 1.81 0) (stroke (width 0.12) (type solid)) (layer "F.SilkS"))
  (fp_line (start 8.35 1.37) (end 8.35 -1.37) (stroke (width 0.12) (type solid)) (layer "F.SilkS"))
  (fp_line (start 1.81 1.37) (end 8.35 1.37) (stroke (width 0.12) (type solid)) (layer "F.SilkS"))
  (pad "1" thru_hole circle (at 0 0 90) (size 1.6 1.6) (drill 0.8) (layers "*.Cu" "*.Mask") (remove_unused_layers no) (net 32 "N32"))
  (pad "2" thru_hole oval (at 10.16 0 90) (size 1.6 1.6) (drill 0.8) (layers "*.Cu" "*.Mask") (remove_unused_layers no) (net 15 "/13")))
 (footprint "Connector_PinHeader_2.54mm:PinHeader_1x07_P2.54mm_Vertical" (layer "F.Cu") (at 146.92 93.5 90)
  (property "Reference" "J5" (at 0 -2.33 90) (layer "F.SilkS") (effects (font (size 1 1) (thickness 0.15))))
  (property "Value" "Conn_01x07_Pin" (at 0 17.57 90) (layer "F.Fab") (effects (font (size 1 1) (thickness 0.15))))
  (fp_line (start -1.33 -1.33) (end 0 -1.33) (stroke (width 0.12) (type solid)) (layer "F.SilkS"))
  (fp_line (start -1.33 0) (end -1.33 -1.33) (stroke (width 0.12) (type solid)) (layer "F.SilkS"))
  (fp_line (start 1.33 1.27) (end 1.33 16.57) (stroke (width 0.12) (type solid)) (layer "F.SilkS"))
  (fp_line (start -1.33 1.27) (end 1.33 1.27) (stroke (width 0.12) (type solid)) (layer "F.SilkS"))
  (fp_line (start -1.33 1.27) (end -1.33 16.57) (stroke (width 0.12) (type solid)) (layer "F.SilkS"))
  (fp_line (start -1.33 16.57) (end 1.33 16.57) (stroke (width 0.12) (type solid)) (layer "F.SilkS"))
  (pad "1" thru_hole rect (at 0 0 90) (size 1.7 1.7) (drill 1) (layers "*.Cu" "*.Mask") (remove_unused_layers no) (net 6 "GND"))
  (pad "2" thru_hole oval (at 0 2.54 90) (size 1.7 1.7) (drill 1) (layers "*.Cu" "*.Mask") (remove_unused_layers no) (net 5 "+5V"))
  (pad "3" thru_hole oval (at 0 5.08 90) (size 1.7 1.7) (drill 1) (layers "*.Cu" "*.Mask") (remove_unused_layers no) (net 8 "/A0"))
  (pad "4" thru_hole oval (at 0 7.62 90) (size 1.7 1.7) (drill 1) (layers "*.Cu" "*.Mask") (remove_unused_layers no) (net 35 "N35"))
  (pad "5" thru_hole oval (at 0 10.16 90) (size 1.7 1.7) (drill 1) (layers "*.Cu" "*.Mask") (remove_unused_layers no) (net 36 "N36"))
  (pad "6" thru_hole oval (at 0 12.7 90) (size 1.7 1.7) (drill 1) (layers "*.Cu" "*.Mask") (remove_unused_layers no) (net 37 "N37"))
  (pad "7" thru_hole oval (at 0 15.24 90) (size 1.7 1.7) (drill 1) (layers "*.Cu" "*.Mask") (remove_unused_layers no) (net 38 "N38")))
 (gr_line (start 166.04 59.36) (end 168.58 61.9) (stroke (width 0.15) (type solid)) (layer "Edge.Cuts"))
 (gr_line (start 100 99.238) (end 100 47.422) (stroke (width 0.15) (type solid)) (layer "Edge.Cuts"))
 (gr_line (start 168.58 61.9) (end 168.58 96.19) (stroke (width 0.15) (type solid)) (layer "Edge.Cuts"))
 (gr_line (start 165.278 100) (end 100.762 100) (stroke (width 0.15) (type solid)) (layer "Edge.Cuts"))
 (gr_line (start 100.762 46.66) (end 163.5 46.66) (stroke (width 0.15) (type solid)) (layer "Edge.Cuts"))
 (gr_arc (start 100.762 100) (mid 100.223185 99.776815) (end 100 99.238) (stroke (width 0.15) (type solid)) (layer "Edge.Cuts"))
 (gr_line (start 168.58 96.19) (end 166.04 98.73) (stroke (width 0.15) (type solid)) (layer "Edge.Cuts"))
 (gr_line (start 163.5 46.66) (end 166.04 49.2) (stroke (width 0.15) (type solid)) (layer "Edge.Cuts"))
 (gr_arc (start 166.04 99.238) (mid 165.816815 99.776815) (end 165.278 100) (stroke (width 0.15) (type solid)) (layer "Edge.Cuts"))
 (gr_line (start 166.04 49.2) (end 166.04 59.36) (stroke (width 0.15) (type solid)) (layer "Edge.Cuts"))
 (gr_line (start 166.04 98.73) (end 166.04 99.238) (stroke (width 0.15) (type solid)) (layer "Edge.Cuts"))
 (gr_arc (start 100 47.422) (mid 100.223185 46.883185) (end 100.762 46.66) (stroke (width 0.15) (type solid)) (layer "Edge.Cuts"))
 (segment (start 146.92 93.5) (end 143.3 93.5) (width 1) (layer "F.Cu") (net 6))
 (segment (start 146.92 93.5) (end 147 93.5) (width 0.25) (layer "F.Cu") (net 6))
 (segment (start 143.3 93.5) (end 140.64 96.16) (width 1) (layer "F.Cu") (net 6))
 (segment (start 140.64 96.257919) (end 140.64 97.46) (width 1) (layer "F.Cu") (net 6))
 (segment (start 147 93.5) (end 147 93.64) (width 0.25) (layer "F.Cu") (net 6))
 (segment (start 137.982081 93.6) (end 140.64 96.257919) (width 1) (layer "F.Cu") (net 6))
 (segment (start 105.4 93.6) (end 137.982081 93.6) (width 1) (layer "F.Cu") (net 6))
 (segment (start 140.64 96.16) (end 140.64 97.46) (width 1) (layer "F.Cu") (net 6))
 (segment (start 138.1 97.46) (end 138.04 97.46) (width 0.25) (layer "F.Cu") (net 5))
 (segment (start 149.46 94.54) (end 149.46 93.5) (width 1) (layer "F.Cu") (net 5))
 (segment (start 138.04 97.46) (end 138 97.5) (width 0.25) (layer "F.Cu") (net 5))
 (segment (start 140.04 99.4) (end 147.379874 99.4) (width 1) (layer "F.Cu") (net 5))
 (segment (start 138.1 97.46) (end 140.04 99.4) (width 1) (layer "F.Cu") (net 5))
 (segment (start 147.379874 99.4) (end 148.291469 98.488405) (width 1) (layer "F.Cu") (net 5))
 (segment (start 148.291469 98.488405) (end 148.291469 95.708531) (width 1) (layer "F.Cu") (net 5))
 (segment (start 148.291469 95.708531) (end 149.46 94.54) (width 1) (layer "F.Cu") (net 5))
 (segment (start 150.8 97.46) (end 150.8 95.61) (width 1) (layer "F.Cu") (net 8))
 (segment (start 150.8 95.61) (end 152 94.41) (width 1) (layer "F.Cu") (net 8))
 (segment (start 152 94.41) (end 152 93.5) (width 1) (layer "F.Cu") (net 8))
 (segment (start 128.956 49.644) (end 128.956 49.2) (width 1) (layer "F.Cu") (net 15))
 (segment (start 114.6 66.52) (end 114.6 64) (width 1) (layer "F.Cu") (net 15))
 (segment (start 114.6 64) (end 128.956 49.644) (width 1) (layer "F.Cu") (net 15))
 (segment (start 131.496 50.096) (end 131.496 49.2) (width 1) (layer "F.Cu") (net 16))
 (segment (start 120.4 61.4) (end 131.6 50.2) (width 1) (layer "F.Cu") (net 16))
 (segment (start 142.2 89.6) (end 121.4 89.6) (width 1) (layer "F.Cu") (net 16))
 (segment (start 146.36 85.44) (end 142.2 89.6) (width 1) (layer "F.Cu") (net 16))
 (segment (start 146.36 79.64) (end 146.36 85.44) (width 1) (layer "F.Cu") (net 16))
 (segment (start 131.6 50.2) (end 131.496 50.096) (width 1) (layer "F.Cu") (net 16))
 (segment (start 121.4 89.6) (end 120.4 88.6) (width 1) (layer "F.Cu") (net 16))
 (segment (start 120.4 88.6) (end 120.4 61.4) (width 1) (layer "F.Cu") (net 16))
 (segment (start 132.8 59.8) (end 140.4 52.2) (width 1) (layer "F.Cu") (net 20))
 (segment (start 141.656 50.744) (end 141.656 49.2) (width 1) (layer "F.Cu") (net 20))
 (segment (start 140.4 52.2) (end 140.4 52) (width 1) (layer "F.Cu") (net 20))
 (segment (start 132.8 65.6) (end 132.8 59.8) (width 1) (layer "F.Cu") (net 20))
 (segment (start 140.4 52) (end 141.656 50.744) (width 1) (layer "F.Cu") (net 20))
 (segment (start 136.04 79.64) (end 136.2 79.64) (width 1) (layer "F.Cu") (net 20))
 (segment (start 136.2 69) (end 132.8 65.6) (width 1) (layer "F.Cu") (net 20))
 (segment (start 136.04 79.64) (end 136 79.6) (width 1) (layer "F.Cu") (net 20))
 (segment (start 136.2 79.64) (end 136.2 69) (width 1) (layer "F.Cu") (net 20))
 (segment (start 142.592103 53.607898) (end 142.592103 52.327897) (width 1) (layer "F.Cu") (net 21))
 (segment (start 142.592103 52.327897) (end 145.72 49.2) (width 1) (layer "F.Cu") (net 21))
 (segment (start 143.82 83.78) (end 139.8 87.8) (width 1) (layer "F.Cu") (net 17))
 (segment (start 143.82 79.64) (end 143.82 83.78) (width 1) (layer "F.Cu") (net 17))
 (segment (start 139.8 87.8) (end 123.6 87.8) (width 1) (layer "F.Cu") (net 17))
 (segment (start 123.6 60.8) (end 134.036 50.364) (width 1) (layer "F.Cu") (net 17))
 (segment (start 134.036 50.364) (end 134.036 49.2) (width 1) (layer "F.Cu") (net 17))
 (segment (start 123.6 87.8) (end 123.6 60.8) (width 1) (layer "F.Cu") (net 17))
 (segment (start 127.8 59.2) (end 136.576 50.424) (width 1) (layer "F.Cu") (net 18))
 (segment (start 141.28 79.64) (end 141.28 82.32) (width 1) (layer "F.Cu") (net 18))
 (segment (start 130.6 85.8) (end 127.8 83) (width 1) (layer "F.Cu") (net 18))
 (segment (start 136.576 50.424) (end 136.576 49.2) (width 1) (layer "F.Cu") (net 18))
 (segment (start 137.8 85.8) (end 130.6 85.8) (width 1) (layer "F.Cu") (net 18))
 (segment (start 141.28 82.32) (end 137.8 85.8) (width 1) (layer "F.Cu") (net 18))
 (segment (start 127.8 83) (end 127.8 59.2) (width 1) (layer "F.Cu") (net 18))
 (segment (start 132.8 71) (end 130.4 68.6) (width 1) (layer "F.Cu") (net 19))
 (segment (start 132.8 83) (end 132.8 71) (width 1) (layer "F.Cu") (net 19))
 (segment (start 133 83.2) (end 132.8 83) (width 1) (layer "F.Cu") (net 19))
 (segment (start 139.116 50.884) (end 139.116 49.2) (width 1) (layer "F.Cu") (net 19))
 (segment (start 138.74 81.66) (end 137.2 83.2) (width 1) (layer "F.Cu") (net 19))
 (segment (start 138.74 79.64) (end 138.74 81.66) (width 1) (layer "F.Cu") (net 19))
 (segment (start 130.4 59.6) (end 139.116 50.884) (width 1) (layer "F.Cu") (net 19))
 (segment (start 137.2 83.2) (end 133 83.2) (width 1) (layer "F.Cu") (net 19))
 (segment (start 130.4 68.6) (end 130.4 59.6) (width 1) (layer "F.Cu") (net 19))
 (segment (start 154.392103 52.807898) (end 153.34 51.755795) (width 1) (layer "F.Cu") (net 24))
 (segment (start 153.34 51.755795) (end 153.34 49.2) (width 1) (layer "F.Cu") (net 24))
 (segment (start 148.9 64.4) (end 165 64.4) (width 1) (layer "F.Cu") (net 26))
 (segment (start 165.4 60.2) (end 165.4 57.2) (width 1) (layer "F.Cu") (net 26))
 (segment (start 165 64.4) (end 167.3 62.1) (width 1) (layer "F.Cu") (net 26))
 (segment (start 165.4 57.2) (end 158.42 50.22) (width 1) (layer "F.Cu") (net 26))
 (segment (start 158.42 50.22) (end 158.42 49.2) (width 1) (layer "F.Cu") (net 26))
 (segment (start 167.3 62.1) (end 165.4 60.2) (width 1) (layer "F.Cu") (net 26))
 (segment (start 142.6 57.07868) (end 148.26 51.41868) (width 1) (layer "F.Cu") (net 22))
 (segment (start 138.74 63.26) (end 142.6 59.4) (width 1) (layer "F.Cu") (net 22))
 (segment (start 142.6 59.4) (end 142.6 57.07868) (width 1) (layer "F.Cu") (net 22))
 (segment (start 138.74 64.4) (end 138.74 63.26) (width 1) (layer "F.Cu") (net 22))
 (segment (start 148.26 51.41868) (end 148.26 49.2) (width 1) (layer "F.Cu") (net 22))
 (segment (start 150.8 51.8) (end 150.8 49.2) (width 1) (layer "F.Cu") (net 23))
 (segment (start 144.6 60) (end 144.6 58) (width 1) (layer "F.Cu") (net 23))
 (segment (start 141.28 64.4) (end 141.28 63.32) (width 1) (layer "F.Cu") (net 23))
 (segment (start 141.28 63.32) (end 144.6 60) (width 1) (layer "F.Cu") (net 23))
 (segment (start 141.28 64.4) (end 141.4 64.4) (width 1) (layer "F.Cu") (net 23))
 (segment (start 144.6 58) (end 150.8 51.8) (width 1) (layer "F.Cu") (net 23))
 (segment (start 155.88 50.68) (end 155.88 49.2) (width 1) (layer "F.Cu") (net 25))
 (segment (start 163.2 60.6) (end 163.2 58) (width 1) (layer "F.Cu") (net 25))
 (segment (start 163.2 58) (end 155.88 50.68) (width 1) (layer "F.Cu") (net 25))
 (segment (start 145.54 97.46) (end 145.5 97.5) (width 0.25) (layer "F.Cu") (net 7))
 (segment (start 145.72 97.46) (end 145.54 97.46) (width 0.25) (layer "F.Cu") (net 7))
 (segment (start 136.2 64.4) (end 136.2 61.584205) (width 1) (layer "F.Cu") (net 29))
 (segment (start 102.2 49.05) (end 102.25 49.05) (width 0.25) (layer "F.Cu") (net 29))
 (segment (start 136.2 61.584205) (end 135.407898 60.792103) (width 1) (layer "F.Cu") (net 29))
 (segment (start 151.44 62.2) (end 153.04 60.6) (width 1) (layer "F.Cu") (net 33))
 (segment (start 146.36 63.64) (end 147.8 62.2) (width 1) (layer "F.Cu") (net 33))
 (segment (start 147.8 62.2) (end 151.44 62.2) (width 1) (layer "F.Cu") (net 33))
 (segment (start 146.36 64.4) (end 146.36 63.64) (width 1) (layer "F.Cu") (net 33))
 (segment (start 147.207898 60.192102) (end 147.207898 59.992103) (width 1) (layer "F.Cu") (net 34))
 (segment (start 143.82 64.4) (end 143.82 63.58) (width 1) (layer "F.Cu") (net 34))
 (segment (start 143.82 63.58) (end 147.207898 60.192102) (width 1) (layer "F.Cu") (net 34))
 (segment (start 143 91.6) (end 148 86.6) (width 1) (layer "F.Cu") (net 32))
 (segment (start 118 89) (end 120.6 91.6) (width 1) (layer "F.Cu") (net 32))
 (segment (start 148.2 86.6) (end 148.9 85.9) (width 1) (layer "F.Cu") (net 32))
 (segment (start 148.9 85.9) (end 148.9 79.64) (width 1) (layer "F.Cu") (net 32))
 (segment (start 114.6 76.68) (end 118 80.08) (width 1) (layer "F.Cu") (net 32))
 (segment (start 118 80.08) (end 118 89) (width 1) (layer "F.Cu") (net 32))
 (segment (start 120.6 91.6) (end 143 91.6) (width 1) (layer "F.Cu") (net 32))
 (segment (start 148 86.6) (end 148.2 86.6) (width 1) (layer "F.Cu") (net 32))
 (segment (start 107.7 89.1) (end 101.9 89.1) (width 1) (layer "F.Cu") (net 31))
 (segment (start 110 91.4) (end 107.7 89.1) (width 1) (layer "F.Cu") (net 31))
 (segment (start 116.4 91.4) (end 110 91.4) (width 1) (layer "F.Cu") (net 31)))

